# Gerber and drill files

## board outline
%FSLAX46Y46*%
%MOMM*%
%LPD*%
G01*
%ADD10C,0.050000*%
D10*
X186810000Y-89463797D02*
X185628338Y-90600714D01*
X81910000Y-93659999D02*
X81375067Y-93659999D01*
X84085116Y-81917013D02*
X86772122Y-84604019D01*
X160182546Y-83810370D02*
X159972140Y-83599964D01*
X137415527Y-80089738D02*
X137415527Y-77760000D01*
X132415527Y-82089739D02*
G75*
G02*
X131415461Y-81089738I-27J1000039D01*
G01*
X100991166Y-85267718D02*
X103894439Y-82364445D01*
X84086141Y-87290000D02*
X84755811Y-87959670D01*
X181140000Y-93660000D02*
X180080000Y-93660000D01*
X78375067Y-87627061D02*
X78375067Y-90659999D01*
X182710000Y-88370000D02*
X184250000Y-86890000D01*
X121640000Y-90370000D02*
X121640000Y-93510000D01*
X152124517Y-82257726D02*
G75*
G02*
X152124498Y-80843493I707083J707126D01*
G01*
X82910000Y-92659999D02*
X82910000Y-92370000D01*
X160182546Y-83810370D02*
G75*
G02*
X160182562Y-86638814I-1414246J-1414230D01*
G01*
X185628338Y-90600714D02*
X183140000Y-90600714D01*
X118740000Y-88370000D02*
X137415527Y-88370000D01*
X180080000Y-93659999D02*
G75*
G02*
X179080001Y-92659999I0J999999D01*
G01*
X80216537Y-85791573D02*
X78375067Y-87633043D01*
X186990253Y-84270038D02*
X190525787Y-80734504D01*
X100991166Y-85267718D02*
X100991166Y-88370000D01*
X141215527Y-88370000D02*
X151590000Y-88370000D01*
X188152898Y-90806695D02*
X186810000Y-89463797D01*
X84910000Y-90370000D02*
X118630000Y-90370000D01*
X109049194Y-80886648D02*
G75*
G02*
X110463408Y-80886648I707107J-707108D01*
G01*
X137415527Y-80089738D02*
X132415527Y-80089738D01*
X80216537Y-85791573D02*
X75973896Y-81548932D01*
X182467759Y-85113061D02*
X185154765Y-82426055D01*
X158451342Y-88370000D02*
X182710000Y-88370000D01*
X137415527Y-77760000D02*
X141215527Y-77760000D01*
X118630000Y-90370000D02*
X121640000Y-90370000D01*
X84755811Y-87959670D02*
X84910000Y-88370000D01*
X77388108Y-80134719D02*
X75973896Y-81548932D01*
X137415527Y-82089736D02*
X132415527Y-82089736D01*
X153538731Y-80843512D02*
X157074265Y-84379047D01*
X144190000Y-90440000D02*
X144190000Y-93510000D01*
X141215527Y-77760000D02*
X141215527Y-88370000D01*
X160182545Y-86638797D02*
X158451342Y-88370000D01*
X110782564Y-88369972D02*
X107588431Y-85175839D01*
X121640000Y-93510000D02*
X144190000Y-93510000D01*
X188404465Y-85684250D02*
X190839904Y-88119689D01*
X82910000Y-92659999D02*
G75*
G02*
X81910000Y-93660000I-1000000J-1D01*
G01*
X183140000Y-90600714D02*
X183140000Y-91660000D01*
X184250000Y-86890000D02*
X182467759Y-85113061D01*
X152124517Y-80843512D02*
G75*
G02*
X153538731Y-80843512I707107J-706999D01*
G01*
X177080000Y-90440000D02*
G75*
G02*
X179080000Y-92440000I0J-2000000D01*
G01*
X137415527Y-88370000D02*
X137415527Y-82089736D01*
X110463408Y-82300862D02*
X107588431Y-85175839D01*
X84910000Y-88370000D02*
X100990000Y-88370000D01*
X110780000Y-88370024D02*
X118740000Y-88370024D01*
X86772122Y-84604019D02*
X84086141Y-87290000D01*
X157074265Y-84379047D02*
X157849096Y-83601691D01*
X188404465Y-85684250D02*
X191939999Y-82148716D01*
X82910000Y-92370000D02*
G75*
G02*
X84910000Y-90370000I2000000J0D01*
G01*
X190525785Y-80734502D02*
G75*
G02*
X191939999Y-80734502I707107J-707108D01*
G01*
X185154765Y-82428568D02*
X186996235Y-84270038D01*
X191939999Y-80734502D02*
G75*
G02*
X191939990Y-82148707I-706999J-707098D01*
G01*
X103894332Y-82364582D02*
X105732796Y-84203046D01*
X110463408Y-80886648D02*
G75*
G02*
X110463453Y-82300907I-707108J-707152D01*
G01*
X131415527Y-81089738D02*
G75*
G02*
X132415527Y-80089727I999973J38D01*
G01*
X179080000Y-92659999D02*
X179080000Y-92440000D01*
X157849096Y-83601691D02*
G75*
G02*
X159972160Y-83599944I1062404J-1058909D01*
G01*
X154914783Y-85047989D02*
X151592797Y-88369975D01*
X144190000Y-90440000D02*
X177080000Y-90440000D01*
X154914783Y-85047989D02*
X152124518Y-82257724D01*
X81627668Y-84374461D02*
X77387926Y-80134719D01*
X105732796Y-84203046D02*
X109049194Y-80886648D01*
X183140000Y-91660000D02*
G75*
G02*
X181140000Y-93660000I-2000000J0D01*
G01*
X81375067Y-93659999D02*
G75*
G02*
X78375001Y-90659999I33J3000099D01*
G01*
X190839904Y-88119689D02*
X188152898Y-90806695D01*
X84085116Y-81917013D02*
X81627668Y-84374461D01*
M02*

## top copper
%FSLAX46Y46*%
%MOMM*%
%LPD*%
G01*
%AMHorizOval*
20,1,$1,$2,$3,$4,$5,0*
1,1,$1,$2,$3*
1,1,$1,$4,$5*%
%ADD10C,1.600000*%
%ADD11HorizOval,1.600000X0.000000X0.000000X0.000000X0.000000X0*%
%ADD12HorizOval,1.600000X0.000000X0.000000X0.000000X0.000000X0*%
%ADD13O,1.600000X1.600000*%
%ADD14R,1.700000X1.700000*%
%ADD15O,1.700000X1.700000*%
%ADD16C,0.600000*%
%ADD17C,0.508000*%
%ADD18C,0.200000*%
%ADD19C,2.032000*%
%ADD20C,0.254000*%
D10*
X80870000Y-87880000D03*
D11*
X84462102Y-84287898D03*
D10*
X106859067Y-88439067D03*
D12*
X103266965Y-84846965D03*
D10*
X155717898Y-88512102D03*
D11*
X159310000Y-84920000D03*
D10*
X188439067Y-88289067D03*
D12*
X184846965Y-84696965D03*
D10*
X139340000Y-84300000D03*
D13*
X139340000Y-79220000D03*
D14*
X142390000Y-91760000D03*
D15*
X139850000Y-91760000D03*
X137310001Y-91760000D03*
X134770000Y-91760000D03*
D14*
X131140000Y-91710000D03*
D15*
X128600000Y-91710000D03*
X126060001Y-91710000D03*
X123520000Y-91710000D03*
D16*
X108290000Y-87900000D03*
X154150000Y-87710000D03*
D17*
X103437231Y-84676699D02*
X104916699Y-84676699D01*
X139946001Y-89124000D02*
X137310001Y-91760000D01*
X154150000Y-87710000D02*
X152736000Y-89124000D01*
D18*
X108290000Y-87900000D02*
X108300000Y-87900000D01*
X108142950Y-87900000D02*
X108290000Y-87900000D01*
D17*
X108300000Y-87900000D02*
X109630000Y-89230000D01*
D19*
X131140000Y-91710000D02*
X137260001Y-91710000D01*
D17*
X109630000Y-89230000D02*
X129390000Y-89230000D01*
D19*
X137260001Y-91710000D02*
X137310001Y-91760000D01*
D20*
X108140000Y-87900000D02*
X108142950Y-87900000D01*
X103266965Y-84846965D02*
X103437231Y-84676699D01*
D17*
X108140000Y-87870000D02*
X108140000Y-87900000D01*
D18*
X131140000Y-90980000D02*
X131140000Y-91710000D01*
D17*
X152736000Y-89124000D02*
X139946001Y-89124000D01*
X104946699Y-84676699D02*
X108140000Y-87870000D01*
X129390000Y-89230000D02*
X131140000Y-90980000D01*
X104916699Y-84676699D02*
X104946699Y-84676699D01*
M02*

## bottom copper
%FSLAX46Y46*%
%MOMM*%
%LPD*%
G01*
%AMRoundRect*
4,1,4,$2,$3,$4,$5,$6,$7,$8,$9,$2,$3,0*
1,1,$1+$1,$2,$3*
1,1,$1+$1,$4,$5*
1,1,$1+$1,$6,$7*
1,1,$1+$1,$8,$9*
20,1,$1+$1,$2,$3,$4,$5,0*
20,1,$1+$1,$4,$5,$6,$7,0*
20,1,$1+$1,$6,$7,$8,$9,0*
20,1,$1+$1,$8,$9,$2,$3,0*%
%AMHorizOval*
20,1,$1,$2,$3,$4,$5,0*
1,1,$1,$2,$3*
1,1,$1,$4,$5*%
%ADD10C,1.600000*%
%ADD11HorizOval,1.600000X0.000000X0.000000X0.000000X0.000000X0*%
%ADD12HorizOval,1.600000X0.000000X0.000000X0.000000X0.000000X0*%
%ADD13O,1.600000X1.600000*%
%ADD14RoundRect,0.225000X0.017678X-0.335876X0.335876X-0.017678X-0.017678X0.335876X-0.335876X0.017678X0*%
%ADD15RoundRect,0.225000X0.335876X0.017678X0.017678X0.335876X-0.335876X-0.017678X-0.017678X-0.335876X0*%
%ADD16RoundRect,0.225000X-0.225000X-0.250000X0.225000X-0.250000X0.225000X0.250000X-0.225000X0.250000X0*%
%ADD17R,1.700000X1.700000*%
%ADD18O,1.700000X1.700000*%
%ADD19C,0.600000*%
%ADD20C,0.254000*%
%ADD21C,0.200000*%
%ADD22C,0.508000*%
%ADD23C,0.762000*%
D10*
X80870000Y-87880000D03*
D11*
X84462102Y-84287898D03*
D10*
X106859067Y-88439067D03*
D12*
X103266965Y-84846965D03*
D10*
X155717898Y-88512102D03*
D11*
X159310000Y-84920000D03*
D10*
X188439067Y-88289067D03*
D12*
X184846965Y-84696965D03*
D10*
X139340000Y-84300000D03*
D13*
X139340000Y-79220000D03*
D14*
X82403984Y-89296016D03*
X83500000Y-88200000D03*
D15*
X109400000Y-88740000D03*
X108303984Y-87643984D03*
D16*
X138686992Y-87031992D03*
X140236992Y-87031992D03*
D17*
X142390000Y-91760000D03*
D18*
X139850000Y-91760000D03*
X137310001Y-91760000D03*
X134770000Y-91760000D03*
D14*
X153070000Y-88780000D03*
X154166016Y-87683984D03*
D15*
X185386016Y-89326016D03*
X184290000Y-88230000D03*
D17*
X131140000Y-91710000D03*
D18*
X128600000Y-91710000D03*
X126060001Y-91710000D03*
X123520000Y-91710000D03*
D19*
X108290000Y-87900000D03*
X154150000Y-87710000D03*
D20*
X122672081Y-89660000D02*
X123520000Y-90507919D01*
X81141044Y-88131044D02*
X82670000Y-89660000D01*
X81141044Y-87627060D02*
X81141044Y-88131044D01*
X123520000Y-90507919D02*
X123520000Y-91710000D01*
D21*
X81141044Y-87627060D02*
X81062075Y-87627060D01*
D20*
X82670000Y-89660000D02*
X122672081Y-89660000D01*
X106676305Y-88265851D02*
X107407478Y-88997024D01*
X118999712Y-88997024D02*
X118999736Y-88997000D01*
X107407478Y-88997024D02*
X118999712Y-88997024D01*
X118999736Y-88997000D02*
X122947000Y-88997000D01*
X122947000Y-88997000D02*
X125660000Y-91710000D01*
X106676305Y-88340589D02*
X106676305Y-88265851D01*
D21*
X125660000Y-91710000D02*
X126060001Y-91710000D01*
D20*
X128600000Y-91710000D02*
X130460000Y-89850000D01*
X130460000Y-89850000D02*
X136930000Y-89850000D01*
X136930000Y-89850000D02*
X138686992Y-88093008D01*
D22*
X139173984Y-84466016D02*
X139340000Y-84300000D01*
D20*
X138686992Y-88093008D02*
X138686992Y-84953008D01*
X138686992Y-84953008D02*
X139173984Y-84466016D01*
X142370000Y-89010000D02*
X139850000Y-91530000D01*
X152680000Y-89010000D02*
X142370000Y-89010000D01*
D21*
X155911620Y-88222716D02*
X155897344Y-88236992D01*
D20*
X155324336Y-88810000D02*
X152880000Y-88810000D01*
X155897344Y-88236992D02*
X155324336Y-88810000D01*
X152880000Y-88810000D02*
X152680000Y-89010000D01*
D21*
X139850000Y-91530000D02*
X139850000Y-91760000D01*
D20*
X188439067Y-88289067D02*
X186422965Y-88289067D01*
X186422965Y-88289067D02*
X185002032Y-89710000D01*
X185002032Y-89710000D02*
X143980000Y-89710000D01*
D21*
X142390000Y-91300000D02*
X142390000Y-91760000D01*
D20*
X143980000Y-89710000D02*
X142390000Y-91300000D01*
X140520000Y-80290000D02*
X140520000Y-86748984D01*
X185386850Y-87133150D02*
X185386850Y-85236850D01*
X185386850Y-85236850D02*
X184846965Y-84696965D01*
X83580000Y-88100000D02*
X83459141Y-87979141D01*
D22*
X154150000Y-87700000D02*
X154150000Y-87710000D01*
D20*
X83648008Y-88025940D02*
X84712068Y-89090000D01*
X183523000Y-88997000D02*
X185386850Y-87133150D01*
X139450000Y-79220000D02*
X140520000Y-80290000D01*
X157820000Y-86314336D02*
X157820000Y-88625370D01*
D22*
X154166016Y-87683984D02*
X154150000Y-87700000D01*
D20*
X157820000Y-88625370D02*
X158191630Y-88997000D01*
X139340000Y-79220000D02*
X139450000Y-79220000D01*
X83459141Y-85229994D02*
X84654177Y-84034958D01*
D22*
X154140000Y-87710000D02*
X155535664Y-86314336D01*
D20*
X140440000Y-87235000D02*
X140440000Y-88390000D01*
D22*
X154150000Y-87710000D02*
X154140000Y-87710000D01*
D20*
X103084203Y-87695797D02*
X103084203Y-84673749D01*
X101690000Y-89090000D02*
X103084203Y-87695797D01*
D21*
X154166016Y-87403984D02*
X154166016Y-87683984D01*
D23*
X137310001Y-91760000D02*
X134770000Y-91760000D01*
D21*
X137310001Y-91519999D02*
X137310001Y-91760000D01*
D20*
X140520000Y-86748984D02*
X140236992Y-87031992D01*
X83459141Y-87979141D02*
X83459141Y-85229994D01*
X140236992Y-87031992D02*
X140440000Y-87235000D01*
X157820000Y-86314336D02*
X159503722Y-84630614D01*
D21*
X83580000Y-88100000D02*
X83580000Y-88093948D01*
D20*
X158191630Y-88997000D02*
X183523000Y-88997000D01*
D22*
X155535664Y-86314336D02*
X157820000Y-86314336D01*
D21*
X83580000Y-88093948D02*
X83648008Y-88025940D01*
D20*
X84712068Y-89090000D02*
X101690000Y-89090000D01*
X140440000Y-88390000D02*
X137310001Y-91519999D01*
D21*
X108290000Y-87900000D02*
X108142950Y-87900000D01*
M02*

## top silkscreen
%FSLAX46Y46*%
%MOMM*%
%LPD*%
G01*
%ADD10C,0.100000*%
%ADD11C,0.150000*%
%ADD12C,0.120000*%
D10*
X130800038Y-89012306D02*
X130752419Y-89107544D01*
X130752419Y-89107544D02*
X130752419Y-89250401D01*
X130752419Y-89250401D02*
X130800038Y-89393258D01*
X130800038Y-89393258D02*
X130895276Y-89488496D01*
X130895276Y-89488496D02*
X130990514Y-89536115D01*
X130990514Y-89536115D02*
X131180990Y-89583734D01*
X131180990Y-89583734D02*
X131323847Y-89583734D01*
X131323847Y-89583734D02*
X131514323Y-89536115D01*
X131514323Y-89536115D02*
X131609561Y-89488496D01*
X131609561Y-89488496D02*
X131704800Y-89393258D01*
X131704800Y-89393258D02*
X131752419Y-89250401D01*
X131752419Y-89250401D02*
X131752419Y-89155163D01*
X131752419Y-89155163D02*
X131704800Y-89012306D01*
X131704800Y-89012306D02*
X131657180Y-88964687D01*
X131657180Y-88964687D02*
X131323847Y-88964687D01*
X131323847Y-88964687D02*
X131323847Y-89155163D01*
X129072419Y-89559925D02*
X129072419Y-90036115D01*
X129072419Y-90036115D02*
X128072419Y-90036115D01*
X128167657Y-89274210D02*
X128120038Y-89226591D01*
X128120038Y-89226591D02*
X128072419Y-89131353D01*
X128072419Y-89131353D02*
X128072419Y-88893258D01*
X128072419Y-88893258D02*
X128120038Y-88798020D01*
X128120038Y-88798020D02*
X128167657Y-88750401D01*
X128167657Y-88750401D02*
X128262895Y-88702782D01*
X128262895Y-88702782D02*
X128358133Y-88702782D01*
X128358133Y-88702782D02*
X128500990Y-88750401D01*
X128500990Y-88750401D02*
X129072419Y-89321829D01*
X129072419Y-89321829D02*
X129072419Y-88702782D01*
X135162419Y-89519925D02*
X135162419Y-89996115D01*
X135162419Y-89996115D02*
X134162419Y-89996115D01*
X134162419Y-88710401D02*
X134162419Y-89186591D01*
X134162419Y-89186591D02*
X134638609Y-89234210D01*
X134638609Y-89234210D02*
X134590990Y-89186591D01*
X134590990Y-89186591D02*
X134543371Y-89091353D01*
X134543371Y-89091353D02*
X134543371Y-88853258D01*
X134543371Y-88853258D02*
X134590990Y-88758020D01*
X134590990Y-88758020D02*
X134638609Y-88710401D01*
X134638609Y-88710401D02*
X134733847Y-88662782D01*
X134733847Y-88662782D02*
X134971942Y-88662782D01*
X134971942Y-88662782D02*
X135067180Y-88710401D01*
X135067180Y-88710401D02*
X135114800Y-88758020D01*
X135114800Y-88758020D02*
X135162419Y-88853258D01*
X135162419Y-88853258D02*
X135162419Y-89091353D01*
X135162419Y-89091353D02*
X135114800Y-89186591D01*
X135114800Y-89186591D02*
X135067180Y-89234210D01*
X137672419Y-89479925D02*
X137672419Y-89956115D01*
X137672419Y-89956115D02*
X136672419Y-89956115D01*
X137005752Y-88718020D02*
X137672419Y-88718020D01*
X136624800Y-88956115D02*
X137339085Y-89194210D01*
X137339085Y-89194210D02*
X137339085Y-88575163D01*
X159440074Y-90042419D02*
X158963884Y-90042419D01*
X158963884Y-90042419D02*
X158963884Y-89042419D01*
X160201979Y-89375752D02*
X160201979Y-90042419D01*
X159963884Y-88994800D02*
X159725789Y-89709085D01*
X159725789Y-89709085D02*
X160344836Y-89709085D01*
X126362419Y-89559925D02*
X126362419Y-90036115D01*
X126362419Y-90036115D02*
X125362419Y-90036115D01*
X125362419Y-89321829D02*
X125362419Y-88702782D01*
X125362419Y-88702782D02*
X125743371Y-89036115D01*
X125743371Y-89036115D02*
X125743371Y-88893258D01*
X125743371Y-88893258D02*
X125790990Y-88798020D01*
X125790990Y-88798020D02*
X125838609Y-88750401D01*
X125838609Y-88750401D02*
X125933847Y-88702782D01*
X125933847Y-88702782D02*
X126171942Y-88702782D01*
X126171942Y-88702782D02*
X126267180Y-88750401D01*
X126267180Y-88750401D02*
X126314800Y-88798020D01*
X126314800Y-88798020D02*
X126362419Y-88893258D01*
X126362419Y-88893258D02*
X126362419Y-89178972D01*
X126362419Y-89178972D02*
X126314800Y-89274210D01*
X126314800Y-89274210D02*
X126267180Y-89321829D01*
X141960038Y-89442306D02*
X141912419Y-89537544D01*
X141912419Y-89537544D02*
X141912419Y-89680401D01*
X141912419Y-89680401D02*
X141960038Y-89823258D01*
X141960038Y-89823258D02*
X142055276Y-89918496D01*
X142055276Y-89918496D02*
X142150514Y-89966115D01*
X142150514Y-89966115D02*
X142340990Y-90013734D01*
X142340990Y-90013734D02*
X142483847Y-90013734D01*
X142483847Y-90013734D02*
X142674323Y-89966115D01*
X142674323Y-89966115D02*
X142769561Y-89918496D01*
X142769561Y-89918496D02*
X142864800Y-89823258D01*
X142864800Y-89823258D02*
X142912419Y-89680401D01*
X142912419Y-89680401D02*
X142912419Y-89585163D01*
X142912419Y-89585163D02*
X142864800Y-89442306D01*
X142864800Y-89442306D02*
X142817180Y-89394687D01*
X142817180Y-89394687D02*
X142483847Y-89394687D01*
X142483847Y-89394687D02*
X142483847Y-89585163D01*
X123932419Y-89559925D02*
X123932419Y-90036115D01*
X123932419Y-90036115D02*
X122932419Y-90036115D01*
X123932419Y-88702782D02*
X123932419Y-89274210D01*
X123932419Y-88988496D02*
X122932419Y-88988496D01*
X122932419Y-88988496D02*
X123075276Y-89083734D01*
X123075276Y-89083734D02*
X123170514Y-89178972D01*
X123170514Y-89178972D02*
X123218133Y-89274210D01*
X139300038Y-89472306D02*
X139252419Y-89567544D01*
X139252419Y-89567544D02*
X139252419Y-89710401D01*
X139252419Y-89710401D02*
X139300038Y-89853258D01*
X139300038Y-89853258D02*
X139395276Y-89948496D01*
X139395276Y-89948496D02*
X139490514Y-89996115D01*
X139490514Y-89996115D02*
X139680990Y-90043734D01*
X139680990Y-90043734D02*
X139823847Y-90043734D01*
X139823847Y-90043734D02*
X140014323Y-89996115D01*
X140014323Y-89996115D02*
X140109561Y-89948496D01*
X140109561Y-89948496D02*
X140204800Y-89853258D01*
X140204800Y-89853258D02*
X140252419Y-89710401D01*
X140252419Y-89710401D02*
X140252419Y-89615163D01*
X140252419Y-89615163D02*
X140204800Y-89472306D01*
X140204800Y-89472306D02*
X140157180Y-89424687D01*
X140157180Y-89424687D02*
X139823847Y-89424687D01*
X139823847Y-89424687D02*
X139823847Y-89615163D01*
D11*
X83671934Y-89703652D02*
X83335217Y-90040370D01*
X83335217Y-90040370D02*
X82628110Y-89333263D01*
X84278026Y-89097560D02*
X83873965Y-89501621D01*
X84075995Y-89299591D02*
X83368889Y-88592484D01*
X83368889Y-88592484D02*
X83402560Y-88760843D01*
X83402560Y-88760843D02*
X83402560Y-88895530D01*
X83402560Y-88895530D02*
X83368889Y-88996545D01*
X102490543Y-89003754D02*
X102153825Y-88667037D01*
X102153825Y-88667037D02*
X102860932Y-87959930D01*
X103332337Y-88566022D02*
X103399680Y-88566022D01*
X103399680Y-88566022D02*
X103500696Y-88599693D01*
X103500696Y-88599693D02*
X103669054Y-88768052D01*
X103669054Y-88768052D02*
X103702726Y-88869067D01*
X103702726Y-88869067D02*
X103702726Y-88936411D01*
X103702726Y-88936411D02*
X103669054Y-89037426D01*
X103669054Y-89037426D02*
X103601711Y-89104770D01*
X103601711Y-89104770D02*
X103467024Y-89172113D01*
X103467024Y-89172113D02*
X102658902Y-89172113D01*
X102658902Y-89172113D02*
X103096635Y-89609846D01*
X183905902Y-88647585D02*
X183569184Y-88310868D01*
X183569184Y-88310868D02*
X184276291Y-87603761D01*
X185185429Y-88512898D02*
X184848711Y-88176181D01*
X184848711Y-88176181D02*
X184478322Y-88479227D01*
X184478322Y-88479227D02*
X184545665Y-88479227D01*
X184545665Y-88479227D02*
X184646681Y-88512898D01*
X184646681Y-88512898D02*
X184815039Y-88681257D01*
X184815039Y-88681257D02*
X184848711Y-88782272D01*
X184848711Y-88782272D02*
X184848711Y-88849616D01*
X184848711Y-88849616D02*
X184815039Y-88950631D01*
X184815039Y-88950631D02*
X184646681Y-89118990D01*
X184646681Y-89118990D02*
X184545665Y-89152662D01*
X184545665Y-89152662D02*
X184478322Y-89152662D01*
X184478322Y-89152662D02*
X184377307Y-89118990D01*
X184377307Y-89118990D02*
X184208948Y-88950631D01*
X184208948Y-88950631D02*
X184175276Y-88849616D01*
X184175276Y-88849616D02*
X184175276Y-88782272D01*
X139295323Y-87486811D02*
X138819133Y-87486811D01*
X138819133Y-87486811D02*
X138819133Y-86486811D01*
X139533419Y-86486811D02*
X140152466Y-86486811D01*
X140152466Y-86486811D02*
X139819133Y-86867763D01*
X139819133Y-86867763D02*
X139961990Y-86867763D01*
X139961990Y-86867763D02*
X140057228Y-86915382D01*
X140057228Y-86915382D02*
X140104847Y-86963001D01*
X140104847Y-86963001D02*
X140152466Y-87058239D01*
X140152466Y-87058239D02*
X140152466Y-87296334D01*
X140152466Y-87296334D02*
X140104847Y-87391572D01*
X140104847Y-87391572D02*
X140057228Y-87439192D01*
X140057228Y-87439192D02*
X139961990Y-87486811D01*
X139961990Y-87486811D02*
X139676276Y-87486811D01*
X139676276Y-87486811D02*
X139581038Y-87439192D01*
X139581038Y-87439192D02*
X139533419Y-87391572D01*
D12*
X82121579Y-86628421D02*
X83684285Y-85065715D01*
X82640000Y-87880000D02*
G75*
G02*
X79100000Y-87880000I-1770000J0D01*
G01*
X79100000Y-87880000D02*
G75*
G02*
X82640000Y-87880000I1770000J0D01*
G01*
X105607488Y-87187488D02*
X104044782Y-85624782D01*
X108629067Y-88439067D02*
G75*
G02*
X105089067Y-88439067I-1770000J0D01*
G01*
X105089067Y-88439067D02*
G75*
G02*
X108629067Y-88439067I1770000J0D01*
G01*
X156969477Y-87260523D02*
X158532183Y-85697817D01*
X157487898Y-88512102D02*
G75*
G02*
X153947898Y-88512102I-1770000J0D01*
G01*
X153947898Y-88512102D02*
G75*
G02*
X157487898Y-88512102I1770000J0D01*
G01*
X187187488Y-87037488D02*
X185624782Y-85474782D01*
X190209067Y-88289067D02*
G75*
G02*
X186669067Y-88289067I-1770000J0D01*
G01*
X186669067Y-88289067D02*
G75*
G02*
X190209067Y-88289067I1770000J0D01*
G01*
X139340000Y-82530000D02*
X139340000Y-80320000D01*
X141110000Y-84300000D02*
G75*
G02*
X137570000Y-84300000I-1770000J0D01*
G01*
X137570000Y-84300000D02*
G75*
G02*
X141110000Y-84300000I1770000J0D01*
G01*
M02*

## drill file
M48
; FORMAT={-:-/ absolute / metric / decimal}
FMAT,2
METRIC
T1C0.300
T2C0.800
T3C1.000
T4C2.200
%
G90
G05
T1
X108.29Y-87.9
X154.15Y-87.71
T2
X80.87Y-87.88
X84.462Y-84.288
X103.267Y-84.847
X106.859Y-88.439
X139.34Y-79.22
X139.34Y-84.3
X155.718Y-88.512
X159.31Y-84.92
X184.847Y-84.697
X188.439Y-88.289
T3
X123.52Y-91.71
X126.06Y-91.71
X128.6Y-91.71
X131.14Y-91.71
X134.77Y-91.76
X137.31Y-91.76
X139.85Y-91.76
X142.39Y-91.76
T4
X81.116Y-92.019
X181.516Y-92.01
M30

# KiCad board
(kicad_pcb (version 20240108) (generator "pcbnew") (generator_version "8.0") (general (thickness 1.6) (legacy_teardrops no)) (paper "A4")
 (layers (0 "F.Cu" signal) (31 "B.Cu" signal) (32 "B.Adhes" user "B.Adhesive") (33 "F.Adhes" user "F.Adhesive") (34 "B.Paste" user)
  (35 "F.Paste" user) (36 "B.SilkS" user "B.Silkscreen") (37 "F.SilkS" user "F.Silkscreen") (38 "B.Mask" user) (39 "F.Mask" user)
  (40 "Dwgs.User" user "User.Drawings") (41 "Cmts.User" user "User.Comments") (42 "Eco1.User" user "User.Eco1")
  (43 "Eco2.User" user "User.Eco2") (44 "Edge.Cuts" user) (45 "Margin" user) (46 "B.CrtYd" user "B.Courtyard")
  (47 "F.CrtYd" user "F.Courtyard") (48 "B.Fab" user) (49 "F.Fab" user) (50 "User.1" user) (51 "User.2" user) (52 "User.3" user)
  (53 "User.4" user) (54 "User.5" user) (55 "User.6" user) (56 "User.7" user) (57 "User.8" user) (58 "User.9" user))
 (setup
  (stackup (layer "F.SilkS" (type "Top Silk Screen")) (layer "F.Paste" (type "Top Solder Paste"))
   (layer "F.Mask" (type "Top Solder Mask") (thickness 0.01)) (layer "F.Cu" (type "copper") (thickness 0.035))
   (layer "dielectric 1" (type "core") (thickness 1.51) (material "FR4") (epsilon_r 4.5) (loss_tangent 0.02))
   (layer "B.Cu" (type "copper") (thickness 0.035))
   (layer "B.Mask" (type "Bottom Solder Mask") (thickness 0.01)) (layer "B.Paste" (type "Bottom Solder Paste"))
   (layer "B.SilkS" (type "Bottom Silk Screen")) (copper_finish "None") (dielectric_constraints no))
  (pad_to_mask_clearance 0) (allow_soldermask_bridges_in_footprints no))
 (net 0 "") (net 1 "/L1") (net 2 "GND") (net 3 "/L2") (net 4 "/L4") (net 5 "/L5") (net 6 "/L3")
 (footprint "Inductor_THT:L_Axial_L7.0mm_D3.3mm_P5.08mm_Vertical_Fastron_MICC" (layer "F.Cu") (at 80.87 87.88 45)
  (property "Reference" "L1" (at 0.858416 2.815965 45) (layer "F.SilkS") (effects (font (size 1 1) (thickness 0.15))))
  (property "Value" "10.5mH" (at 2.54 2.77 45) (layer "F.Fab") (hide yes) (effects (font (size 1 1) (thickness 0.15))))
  (fp_line (start 1.77 0) (end 3.98 0) (stroke (width 0.12) (type solid)) (layer "F.SilkS"))
  (fp_circle (center 0 0) (end 1.77 0) (stroke (width 0.12) (type solid)) (fill none) (layer "F.SilkS"))
  (pad "1" thru_hole circle (at 0 0 45) (size 1.6 1.6) (drill 0.8) (layers "*.Cu" "*.Mask") (remove_unused_layers no) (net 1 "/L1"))
  (pad "2" thru_hole oval (at 5.079999 0 45) (size 1.6 1.6) (drill 0.8) (layers "*.Cu" "*.Mask") (remove_unused_layers no) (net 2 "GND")))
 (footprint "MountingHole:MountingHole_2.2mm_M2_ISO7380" (layer "F.Cu") (at 81.115528 92.019237)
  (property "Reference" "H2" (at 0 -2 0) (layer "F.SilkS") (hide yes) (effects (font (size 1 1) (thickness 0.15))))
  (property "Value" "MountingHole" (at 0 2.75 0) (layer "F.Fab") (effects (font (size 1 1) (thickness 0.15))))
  (pad "" np_thru_hole circle (at 0 0) (size 2.2 2.2) (drill 2.2) (layers "*.Cu" "*.Mask")))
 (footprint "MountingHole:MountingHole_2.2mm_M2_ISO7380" (layer "F.Cu") (at 181.515528 92.01)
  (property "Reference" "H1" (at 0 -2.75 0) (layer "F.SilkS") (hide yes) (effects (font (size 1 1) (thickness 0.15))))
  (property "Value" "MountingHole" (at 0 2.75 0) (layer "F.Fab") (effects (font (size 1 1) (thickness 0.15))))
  (pad "" np_thru_hole circle (at 0 0) (size 2.2 2.2) (drill 2.2) (layers "*.Cu" "*.Mask")))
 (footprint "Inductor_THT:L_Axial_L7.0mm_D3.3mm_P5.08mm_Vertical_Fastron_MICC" (layer "F.Cu") (at 106.859067 88.439067 135)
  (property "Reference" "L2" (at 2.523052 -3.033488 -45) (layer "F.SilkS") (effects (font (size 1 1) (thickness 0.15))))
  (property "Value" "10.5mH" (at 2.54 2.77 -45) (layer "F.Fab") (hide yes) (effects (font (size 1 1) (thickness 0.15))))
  (fp_line (start 1.77 0) (end 3.98 0) (stroke (width 0.12) (type solid)) (layer "F.SilkS"))
  (fp_circle (center 0 0) (end 1.77 0) (stroke (width 0.12) (type solid)) (fill none) (layer "F.SilkS"))
  (pad "1" thru_hole circle (at 0 0 135) (size 1.6 1.6) (drill 0.8) (layers "*.Cu" "*.Mask") (remove_unused_layers no) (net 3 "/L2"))
  (pad "2" thru_hole oval (at 5.079999 0 135) (size 1.6 1.6) (drill 0.8) (layers "*.Cu" "*.Mask") (remove_unused_layers no) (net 2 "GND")))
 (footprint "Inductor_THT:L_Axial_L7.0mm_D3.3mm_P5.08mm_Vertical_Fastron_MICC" (layer "F.Cu") (at 155.717898 88.512102 45)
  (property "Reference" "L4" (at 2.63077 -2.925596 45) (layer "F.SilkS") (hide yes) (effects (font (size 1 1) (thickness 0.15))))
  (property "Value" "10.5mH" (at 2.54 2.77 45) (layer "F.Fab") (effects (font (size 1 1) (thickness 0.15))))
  (fp_line (start 1.77 0) (end 3.98 0) (stroke (width 0.12) (type solid)) (layer "F.SilkS"))
  (fp_circle (center 0 0) (end 1.77 0) (stroke (width 0.12) (type solid)) (fill none) (layer "F.SilkS"))
  (pad "1" thru_hole circle (at 0 0 45) (size 1.6 1.6) (drill 0.8) (layers "*.Cu" "*.Mask") (remove_unused_layers no) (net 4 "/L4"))
  (pad "2" thru_hole oval (at 5.079999 0 45) (size 1.6 1.6) (drill 0.8) (layers "*.Cu" "*.Mask") (remove_unused_layers no) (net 2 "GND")))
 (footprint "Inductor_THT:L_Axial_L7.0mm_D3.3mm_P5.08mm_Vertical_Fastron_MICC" (layer "F.Cu") (at 188.439067 88.289067 135)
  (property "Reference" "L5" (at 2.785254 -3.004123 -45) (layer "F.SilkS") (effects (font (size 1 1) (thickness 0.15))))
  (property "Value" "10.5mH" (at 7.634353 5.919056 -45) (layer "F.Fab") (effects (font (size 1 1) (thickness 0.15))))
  (fp_line (start 1.77 0) (end 3.98 0) (stroke (width 0.12) (type solid)) (layer "F.SilkS"))
  (fp_circle (center 0 0) (end 1.77 0) (stroke (width 0.12) (type solid)) (fill none) (layer "F.SilkS"))
  (pad "1" thru_hole circle (at 0 0 135) (size 1.6 1.6) (drill 0.8) (layers "*.Cu" "*.Mask") (remove_unused_layers no) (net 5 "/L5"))
  (pad "2" thru_hole oval (at 5.079999 0 135) (size 1.6 1.6) (drill 0.8) (layers "*.Cu" "*.Mask") (remove_unused_layers no) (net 2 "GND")))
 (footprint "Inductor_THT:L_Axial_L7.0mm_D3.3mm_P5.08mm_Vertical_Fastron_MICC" (layer "F.Cu") (at 139.34 84.3 90)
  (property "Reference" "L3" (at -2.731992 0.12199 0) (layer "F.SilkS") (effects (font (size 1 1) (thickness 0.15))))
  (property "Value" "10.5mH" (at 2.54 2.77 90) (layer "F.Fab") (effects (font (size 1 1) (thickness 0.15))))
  (fp_line (start 1.77 0) (end 3.98 0) (stroke (width 0.12) (type solid)) (layer "F.SilkS"))
  (fp_circle (center 0 0) (end 1.77 0) (stroke (width 0.12) (type solid)) (fill none) (layer "F.SilkS"))
  (pad "1" thru_hole circle (at 0 0 90) (size 1.6 1.6) (drill 0.8) (layers "*.Cu" "*.Mask") (remove_unused_layers no) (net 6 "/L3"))
  (pad "2" thru_hole oval (at 5.08 0 90) (size 1.6 1.6) (drill 0.8) (layers "*.Cu" "*.Mask") (remove_unused_layers no) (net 2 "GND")))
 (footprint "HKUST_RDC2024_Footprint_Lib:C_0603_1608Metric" (layer "B.Cu") (at 82.951992 88.748008 45)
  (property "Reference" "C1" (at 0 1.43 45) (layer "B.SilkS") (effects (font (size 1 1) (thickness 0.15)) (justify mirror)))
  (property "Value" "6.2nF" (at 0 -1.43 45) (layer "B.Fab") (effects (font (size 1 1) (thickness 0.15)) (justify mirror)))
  (pad "1" smd roundrect (at -0.775 0 45) (size 0.9 0.95) (layers "B.Cu" "B.Paste" "B.Mask") (roundrect_rratio 0.25) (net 1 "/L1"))
  (pad "2" smd roundrect (at 0.775 0 45) (size 0.9 0.95) (layers "B.Cu" "B.Paste" "B.Mask") (roundrect_rratio 0.25) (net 2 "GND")))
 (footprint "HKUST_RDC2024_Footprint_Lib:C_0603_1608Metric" (layer "B.Cu") (at 108.851992 88.191992 135)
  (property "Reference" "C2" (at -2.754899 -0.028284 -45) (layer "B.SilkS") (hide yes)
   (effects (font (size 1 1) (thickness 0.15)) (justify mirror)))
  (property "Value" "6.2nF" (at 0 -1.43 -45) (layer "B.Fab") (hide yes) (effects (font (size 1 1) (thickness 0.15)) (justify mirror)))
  (pad "1" smd roundrect (at -0.775 0 135) (size 0.9 0.95) (layers "B.Cu" "B.Paste" "B.Mask") (roundrect_rratio 0.25) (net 3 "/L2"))
  (pad "2" smd roundrect (at 0.775 0 135) (size 0.9 0.95) (layers "B.Cu" "B.Paste" "B.Mask") (roundrect_rratio 0.25) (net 2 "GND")))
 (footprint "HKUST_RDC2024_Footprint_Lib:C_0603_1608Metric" (layer "B.Cu") (at 139.461992 87.031992)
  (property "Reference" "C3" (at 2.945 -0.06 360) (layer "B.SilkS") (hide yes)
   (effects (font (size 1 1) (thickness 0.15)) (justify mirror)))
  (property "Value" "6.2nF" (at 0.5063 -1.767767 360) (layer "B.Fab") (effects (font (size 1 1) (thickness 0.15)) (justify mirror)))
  (pad "1" smd roundrect (at -0.775 0) (size 0.9 0.95) (layers "B.Cu" "B.Paste" "B.Mask") (roundrect_rratio 0.25) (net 6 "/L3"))
  (pad "2" smd roundrect (at 0.775 0) (size 0.9 0.95) (layers "B.Cu" "B.Paste" "B.Mask") (roundrect_rratio 0.25) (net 2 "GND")))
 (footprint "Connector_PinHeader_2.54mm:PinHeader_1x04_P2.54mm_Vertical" (layer "B.Cu") (at 142.39 91.76 90)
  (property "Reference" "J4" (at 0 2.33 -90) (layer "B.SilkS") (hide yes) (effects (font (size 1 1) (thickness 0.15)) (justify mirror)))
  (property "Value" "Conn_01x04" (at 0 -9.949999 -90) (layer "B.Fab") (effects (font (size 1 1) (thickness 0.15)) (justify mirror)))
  (pad "1" thru_hole rect (at 0 0 90) (size 1.7 1.7) (drill 1) (layers "*.Cu" "*.Mask") (remove_unused_layers no) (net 5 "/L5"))
  (pad "2" thru_hole oval (at 0 -2.54 90) (size 1.7 1.7) (drill 1) (layers "*.Cu" "*.Mask") (remove_unused_layers no) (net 4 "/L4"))
  (pad "3" thru_hole oval (at 0 -5.079999 90) (size 1.7 1.7) (drill 1) (layers "*.Cu" "*.Mask") (remove_unused_layers no) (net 2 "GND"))
  (pad "4" thru_hole oval (at 0 -7.62 90) (size 1.7 1.7) (drill 1) (layers "*.Cu" "*.Mask") (remove_unused_layers no) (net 2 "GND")))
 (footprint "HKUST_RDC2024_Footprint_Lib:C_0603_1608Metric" (layer "B.Cu") (at 153.618008 88.231992 45)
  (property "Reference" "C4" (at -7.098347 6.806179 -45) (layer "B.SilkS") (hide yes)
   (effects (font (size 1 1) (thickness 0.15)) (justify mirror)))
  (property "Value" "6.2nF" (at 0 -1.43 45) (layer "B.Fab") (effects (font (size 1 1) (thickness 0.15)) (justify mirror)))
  (pad "1" smd roundrect (at -0.775 0 45) (size 0.9 0.95) (layers "B.Cu" "B.Paste" "B.Mask") (roundrect_rratio 0.25) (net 4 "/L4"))
  (pad "2" smd roundrect (at 0.775 0 45) (size 0.9 0.95) (layers "B.Cu" "B.Paste" "B.Mask") (roundrect_rratio 0.25) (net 2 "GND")))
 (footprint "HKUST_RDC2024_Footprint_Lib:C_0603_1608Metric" (layer "B.Cu") (at 184.838008 88.778008 135)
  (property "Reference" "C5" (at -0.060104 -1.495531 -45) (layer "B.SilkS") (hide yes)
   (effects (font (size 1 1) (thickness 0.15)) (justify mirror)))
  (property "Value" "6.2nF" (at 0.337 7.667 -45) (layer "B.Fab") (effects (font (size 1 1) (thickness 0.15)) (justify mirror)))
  (pad "1" smd roundrect (at -0.775 0 135) (size 0.9 0.95) (layers "B.Cu" "B.Paste" "B.Mask") (roundrect_rratio 0.25) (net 5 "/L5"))
  (pad "2" smd roundrect (at 0.775 0 135) (size 0.9 0.95) (layers "B.Cu" "B.Paste" "B.Mask") (roundrect_rratio 0.25) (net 2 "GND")))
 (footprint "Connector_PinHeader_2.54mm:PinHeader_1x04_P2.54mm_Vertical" (layer "B.Cu") (at 131.14 91.71 90)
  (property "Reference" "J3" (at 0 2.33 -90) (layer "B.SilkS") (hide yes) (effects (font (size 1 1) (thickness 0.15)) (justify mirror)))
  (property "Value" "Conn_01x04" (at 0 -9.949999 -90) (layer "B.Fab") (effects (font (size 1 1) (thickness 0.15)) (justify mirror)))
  (pad "1" thru_hole rect (at 0 0 90) (size 1.7 1.7) (drill 1) (layers "*.Cu" "*.Mask") (remove_unused_layers no) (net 2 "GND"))
  (pad "2" thru_hole oval (at 0 -2.54 90) (size 1.7 1.7) (drill 1) (layers "*.Cu" "*.Mask") (remove_unused_layers no) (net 6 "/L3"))
  (pad "3" thru_hole oval (at 0 -5.079999 90) (size 1.7 1.7) (drill 1) (layers "*.Cu" "*.Mask") (remove_unused_layers no) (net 3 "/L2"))
  (pad "4" thru_hole oval (at 0 -7.62 90) (size 1.7 1.7) (drill 1) (layers "*.Cu" "*.Mask") (remove_unused_layers no) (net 1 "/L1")))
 (gr_line (start 186.81 89.463797) (end 185.628338 90.600714) (stroke (width 0.05) (type default)) (layer "Edge.Cuts"))
 (gr_line (start 81.91 93.659999) (end 81.375067 93.659999) (stroke (width 0.05) (type default)) (layer "Edge.Cuts"))
 (gr_line (start 84.085116 81.917013) (end 86.772122 84.604019) (stroke (width 0.05) (type default)) (layer "Edge.Cuts"))
 (gr_line (start 160.182546 83.81037) (end 159.97214 83.599964) (stroke (width 0.05) (type default)) (layer "Edge.Cuts"))
 (gr_line (start 137.415527 80.089738) (end 137.415527 77.76) (stroke (width 0.05) (type default)) (layer "Edge.Cuts"))
 (gr_arc (start 132.415527 82.089739) (mid 131.70842 81.796845) (end 131.415527 81.089738) (stroke (width 0.05) (type default))
  (layer "Edge.Cuts"))
 (gr_line (start 100.991166 85.267718) (end 103.894439 82.364445) (stroke (width 0.05) (type default)) (layer "Edge.Cuts"))
 (gr_line (start 84.086141 87.29) (end 84.755811 87.95967) (stroke (width 0.05) (type default)) (layer "Edge.Cuts"))
 (gr_line (start 181.14 93.66) (end 180.08 93.66) (stroke (width 0.05) (type default)) (layer "Edge.Cuts"))
 (gr_line (start 78.375067 87.627061) (end 78.375067 90.659999) (stroke (width 0.05) (type default)) (layer "Edge.Cuts"))
 (gr_line (start 182.71 88.37) (end 184.25 86.89) (stroke (width 0.05) (type default)) (layer "Edge.Cuts"))
 (gr_line (start 121.64 90.37) (end 121.64 93.51) (stroke (width 0.05) (type default)) (layer "Edge.Cuts"))
 (gr_arc (start 152.124517 82.257726) (mid 151.831624 81.550619) (end 152.124517 80.843512) (stroke (width 0.05) (type default))
  (layer "Edge.Cuts"))
 (gr_line (start 82.91 92.659999) (end 82.91 92.37) (stroke (width 0.05) (type default)) (layer "Edge.Cuts"))
 (gr_arc (start 160.182546 83.81037) (mid 160.768332 85.224584) (end 160.182545 86.638797) (stroke (width 0.05) (type default))
  (layer "Edge.Cuts"))
 (gr_line (start 185.628338 90.600714) (end 183.14 90.600714) (stroke (width 0.05) (type default)) (layer "Edge.Cuts"))
 (gr_line (start 118.74 88.37) (end 137.415527 88.37) (stroke (width 0.05) (type default)) (layer "Edge.Cuts"))
 (gr_arc (start 180.08 93.659999) (mid 179.372893 93.367106) (end 179.08 92.659999) (stroke (width 0.05) (type default)) (layer "Edge.Cuts"))
 (gr_line (start 80.216537 85.791573) (end 78.375067 87.633043) (stroke (width 0.05) (type default)) (layer "Edge.Cuts"))
 (gr_line (start 186.990253 84.270038) (end 190.525787 80.734504) (stroke (width 0.05) (type default)) (layer "Edge.Cuts"))
 (gr_line (start 100.991166 85.267718) (end 100.991166 88.37) (stroke (width 0.05) (type default)) (layer "Edge.Cuts"))
 (gr_line (start 141.215527 88.37) (end 151.59 88.37) (stroke (width 0.05) (type default)) (layer "Edge.Cuts"))
 (gr_line (start 188.152898 90.806695) (end 186.81 89.463797) (stroke (width 0.05) (type default)) (layer "Edge.Cuts"))
 (gr_line (start 84.91 90.37) (end 118.63 90.37) (stroke (width 0.05) (type default)) (layer "Edge.Cuts"))
 (gr_arc (start 109.049194 80.886648) (mid 109.756301 80.593755) (end 110.463408 80.886648) (stroke (width 0.05) (type default))
  (layer "Edge.Cuts"))
 (gr_line (start 137.415527 80.089738) (end 132.415527 80.089738) (stroke (width 0.05) (type default)) (layer "Edge.Cuts"))
 (gr_line (start 80.216537 85.791573) (end 75.973896 81.548932) (stroke (width 0.05) (type default)) (layer "Edge.Cuts"))
 (gr_line (start 182.467759 85.113061) (end 185.154765 82.426055) (stroke (width 0.05) (type default)) (layer "Edge.Cuts"))
 (gr_line (start 158.451342 88.37) (end 182.71 88.37) (stroke (width 0.05) (type default)) (layer "Edge.Cuts"))
 (gr_line (start 137.415527 77.76) (end 141.215527 77.76) (stroke (width 0.05) (type default)) (layer "Edge.Cuts"))
 (gr_line (start 118.63 90.37) (end 121.64 90.37) (stroke (width 0.05) (type default)) (layer "Edge.Cuts"))
 (gr_line (start 84.755811 87.95967) (end 84.91 88.37) (stroke (width 0.05) (type default)) (layer "Edge.Cuts"))
 (gr_line (start 77.388108 80.134719) (end 75.973896 81.548932) (stroke (width 0.05) (type default)) (layer "Edge.Cuts"))
 (gr_line (start 137.415527 82.089736) (end 132.415527 82.089736) (stroke (width 0.05) (type default)) (layer "Edge.Cuts"))
 (gr_line (start 153.538731 80.843512) (end 157.074265 84.379047) (stroke (width 0.05) (type default)) (layer "Edge.Cuts"))
 (gr_line (start 144.19 90.44) (end 144.19 93.51) (stroke (width 0.05) (type default)) (layer "Edge.Cuts"))
 (gr_line (start 141.215527 77.76) (end 141.215527 88.37) (stroke (width 0.05) (type default)) (layer "Edge.Cuts"))
 (gr_line (start 160.182545 86.638797) (end 158.451342 88.37) (stroke (width 0.05) (type default)) (layer "Edge.Cuts"))
 (gr_line (start 110.782564 88.369972) (end 107.588431 85.175839) (stroke (width 0.05) (type default)) (layer "Edge.Cuts"))
 (gr_line (start 121.64 93.51) (end 144.19 93.51) (stroke (width 0.05) (type default)) (layer "Edge.Cuts"))
 (gr_line (start 188.404465 85.68425) (end 190.839904 88.119689) (stroke (width 0.05) (type default)) (layer "Edge.Cuts"))
 (gr_arc (start 82.91 92.659999) (mid 82.617107 93.367106) (end 81.91 93.659999) (stroke (width 0.05) (type default)) (layer "Edge.Cuts"))
 (gr_line (start 183.14 90.600714) (end 183.14 91.66) (stroke (width 0.05) (type default)) (layer "Edge.Cuts"))
 (gr_line (start 184.25 86.89) (end 182.467759 85.113061) (stroke (width 0.05) (type default)) (layer "Edge.Cuts"))
 (gr_arc (start 152.124517 80.843512) (mid 152.831637 80.550587) (end 153.538731 80.843512) (stroke (width 0.05) (type default))
  (layer "Edge.Cuts"))
 (gr_arc (start 177.08 90.44) (mid 178.494214 91.025786) (end 179.08 92.44) (stroke (width 0.05) (type default)) (layer "Edge.Cuts"))
 (gr_line (start 137.415527 88.37) (end 137.415527 82.089736) (stroke (width 0.05) (type default)) (layer "Edge.Cuts"))
 (gr_line (start 110.463408 82.300862) (end 107.588431 85.175839) (stroke (width 0.05) (type default)) (layer "Edge.Cuts"))
 (gr_line (start 84.91 88.37) (end 100.99 88.37) (stroke (width 0.05) (type default)) (layer "Edge.Cuts"))
 (gr_line (start 110.78 88.370024) (end 118.74 88.370024) (stroke (width 0.05) (type default)) (layer "Edge.Cuts"))
 (gr_line (start 86.772122 84.604019) (end 84.086141 87.29) (stroke (width 0.05) (type default)) (layer "Edge.Cuts"))
 (gr_line (start 157.074265 84.379047) (end 157.849096 83.601691) (stroke (width 0.05) (type default)) (layer "Edge.Cuts"))
 (gr_line (start 188.404465 85.68425) (end 191.939999 82.148716) (stroke (width 0.05) (type default)) (layer "Edge.Cuts"))
 (gr_arc (start 82.91 92.37) (mid 83.495786 90.955786) (end 84.91 90.37) (stroke (width 0.05) (type default)) (layer "Edge.Cuts"))
 (gr_arc (start 190.525785 80.734502) (mid 191.232892 80.441609) (end 191.939999 80.734502) (stroke (width 0.05) (type default))
  (layer "Edge.Cuts"))
 (gr_line (start 185.154765 82.428568) (end 186.996235 84.270038) (stroke (width 0.05) (type default)) (layer "Edge.Cuts"))
 (gr_arc (start 191.939999 80.734502) (mid 192.232924 81.441622) (end 191.939999 82.148716) (stroke (width 0.05) (type default))
  (layer "Edge.Cuts"))
 (gr_line (start 103.894332 82.364582) (end 105.732796 84.203046) (stroke (width 0.05) (type default)) (layer "Edge.Cuts"))
 (gr_arc (start 110.463408 80.886648) (mid 110.756301 81.593755) (end 110.463408 82.300862) (stroke (width 0.05) (type default))
  (layer "Edge.Cuts"))
 (gr_arc (start 131.415527 81.089738) (mid 131.708407 80.3826) (end 132.415527 80.089738) (stroke (width 0.05) (type default))
  (layer "Edge.Cuts"))
 (gr_line (start 179.08 92.659999) (end 179.08 92.44) (stroke (width 0.05) (type default)) (layer "Edge.Cuts"))
 (gr_arc (start 157.849096 83.601691) (mid 158.91026 83.160625) (end 159.97214 83.599964) (stroke (width 0.05) (type default))
  (layer "Edge.Cuts"))
 (gr_line (start 154.914783 85.047989) (end 151.592797 88.369975) (stroke (width 0.05) (type default)) (layer "Edge.Cuts"))
 (gr_line (start 144.19 90.44) (end 177.08 90.44) (stroke (width 0.05) (type default)) (layer "Edge.Cuts"))
 (gr_line (start 154.914783 85.047989) (end 152.124518 82.257724) (stroke (width 0.05) (type default)) (layer "Edge.Cuts"))
 (gr_line (start 81.627668 84.374461) (end 77.387926 80.134719) (stroke (width 0.05) (type default)) (layer "Edge.Cuts"))
 (gr_line (start 105.732796 84.203046) (end 109.049194 80.886648) (stroke (width 0.05) (type default)) (layer "Edge.Cuts"))
 (gr_arc (start 183.14 91.66) (mid 182.554214 93.074214) (end 181.14 93.66) (stroke (width 0.05) (type default)) (layer "Edge.Cuts"))
 (gr_arc (start 81.375067 93.659999) (mid 79.253768 92.781308) (end 78.375067 90.659999) (stroke (width 0.05) (type default))
  (layer "Edge.Cuts"))
 (gr_line (start 190.839904 88.119689) (end 188.152898 90.806695) (stroke (width 0.05) (type default)) (layer "Edge.Cuts"))
 (gr_line (start 84.085116 81.917013) (end 81.627668 84.374461) (stroke (width 0.05) (type default)) (layer "Edge.Cuts"))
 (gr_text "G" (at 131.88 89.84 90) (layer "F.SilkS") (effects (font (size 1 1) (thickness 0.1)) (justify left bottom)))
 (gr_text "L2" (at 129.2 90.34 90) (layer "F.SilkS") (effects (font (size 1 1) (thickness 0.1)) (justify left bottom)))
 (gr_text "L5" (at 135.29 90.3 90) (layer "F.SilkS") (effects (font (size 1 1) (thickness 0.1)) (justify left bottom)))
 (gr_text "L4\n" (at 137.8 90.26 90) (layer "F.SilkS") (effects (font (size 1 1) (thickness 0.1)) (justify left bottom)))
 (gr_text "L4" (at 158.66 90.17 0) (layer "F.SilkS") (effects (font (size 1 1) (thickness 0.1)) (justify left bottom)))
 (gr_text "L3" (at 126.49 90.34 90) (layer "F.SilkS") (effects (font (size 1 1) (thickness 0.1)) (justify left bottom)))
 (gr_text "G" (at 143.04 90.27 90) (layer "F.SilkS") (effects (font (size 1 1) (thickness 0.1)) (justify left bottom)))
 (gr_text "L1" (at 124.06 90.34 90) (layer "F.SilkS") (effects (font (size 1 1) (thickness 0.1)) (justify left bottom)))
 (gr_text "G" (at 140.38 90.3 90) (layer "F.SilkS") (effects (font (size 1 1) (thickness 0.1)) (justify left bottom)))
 (segment (start 122.672081 89.66) (end 123.52 90.507919) (width 0.254) (layer "B.Cu") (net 1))
 (segment (start 81.141044 88.131044) (end 82.67 89.66) (width 0.254) (layer "B.Cu") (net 1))
 (segment (start 81.141044 87.62706) (end 81.141044 88.131044) (width 0.254) (layer "B.Cu") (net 1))
 (segment (start 123.52 90.507919) (end 123.52 91.71) (width 0.254) (layer "B.Cu") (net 1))
 (segment (start 81.141044 87.62706) (end 81.062075 87.62706) (width 0.2) (layer "B.Cu") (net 1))
 (segment (start 82.67 89.66) (end 122.672081 89.66) (width 0.254) (layer "B.Cu") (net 1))
 (segment (start 106.676305 88.265851) (end 107.407478 88.997024) (width 0.254) (layer "B.Cu") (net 3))
 (segment (start 118.999712 88.997024) (end 118.999736 88.997) (width 0.254) (layer "B.Cu") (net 3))
 (segment (start 107.407478 88.997024) (end 118.999712 88.997024) (width 0.254) (layer "B.Cu") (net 3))
 (segment (start 118.999736 88.997) (end 122.947 88.997) (width 0.254) (layer "B.Cu") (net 3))
 (segment (start 122.947 88.997) (end 125.66 91.71) (width 0.254) (layer "B.Cu") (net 3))
 (segment (start 106.676305 88.340589) (end 106.676305 88.265851) (width 0.254) (layer "B.Cu") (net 3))
 (segment (start 125.66 91.71) (end 126.060001 91.71) (width 0.2) (layer "B.Cu") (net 3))
 (segment (start 128.6 91.71) (end 130.46 89.85) (width 0.254) (layer "B.Cu") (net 6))
 (segment (start 130.46 89.85) (end 136.93 89.85) (width 0.254) (layer "B.Cu") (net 6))
 (segment (start 136.93 89.85) (end 138.686992 88.093008) (width 0.254) (layer "B.Cu") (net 6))
 (segment (start 139.173984 84.466016) (end 139.34 84.3) (width 0.508) (layer "B.Cu") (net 6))
 (segment (start 138.686992 88.093008) (end 138.686992 84.953008) (width 0.254) (layer "B.Cu") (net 6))
 (segment (start 138.686992 84.953008) (end 139.173984 84.466016) (width 0.254) (layer "B.Cu") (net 6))
 (segment (start 142.37 89.01) (end 139.85 91.53) (width 0.254) (layer "B.Cu") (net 4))
 (segment (start 152.68 89.01) (end 142.37 89.01) (width 0.254) (layer "B.Cu") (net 4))
 (segment (start 155.91162 88.222716) (end 155.897344 88.236992) (width 0.2) (layer "B.Cu") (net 4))
 (segment (start 155.324336 88.81) (end 152.88 88.81) (width 0.254) (layer "B.Cu") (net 4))
 (segment (start 155.897344 88.236992) (end 155.324336 88.81) (width 0.254) (layer "B.Cu") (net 4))
 (segment (start 152.88 88.81) (end 152.68 89.01) (width 0.254) (layer "B.Cu") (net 4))
 (segment (start 139.85 91.53) (end 139.85 91.76) (width 0.2) (layer "B.Cu") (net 4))
 (segment (start 188.439067 88.289067) (end 186.422965 88.289067) (width 0.254) (layer "B.Cu") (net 5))
 (segment (start 186.422965 88.289067) (end 185.002032 89.71) (width 0.254) (layer "B.Cu") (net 5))
 (segment (start 185.002032 89.71) (end 143.98 89.71) (width 0.254) (layer "B.Cu") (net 5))
 (segment (start 142.39 91.3) (end 142.39 91.76) (width 0.2) (layer "B.Cu") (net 5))
 (segment (start 143.98 89.71) (end 142.39 91.3) (width 0.254) (layer "B.Cu") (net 5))
 (segment (start 103.437231 84.676699) (end 104.916699 84.676699) (width 0.508) (layer "F.Cu") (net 2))
 (segment (start 139.946001 89.124) (end 137.310001 91.76) (width 0.508) (layer "F.Cu") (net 2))
 (segment (start 154.15 87.71) (end 152.736 89.124) (width 0.508) (layer "F.Cu") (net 2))
 (segment (start 108.29 87.9) (end 108.3 87.9) (width 0.2) (layer "F.Cu") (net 2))
 (segment (start 108.14295 87.9) (end 108.29 87.9) (width 0.2) (layer "F.Cu") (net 2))
 (segment (start 108.3 87.9) (end 109.63 89.23) (width 0.508) (layer "F.Cu") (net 2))
 (segment (start 131.14 91.71) (end 137.260001 91.71) (width 2.032) (layer "F.Cu") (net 2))
 (segment (start 109.63 89.23) (end 129.39 89.23) (width 0.508) (layer "F.Cu") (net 2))
 (segment (start 137.260001 91.71) (end 137.310001 91.76) (width 2.032) (layer "F.Cu") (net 2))
 (segment (start 108.14 87.9) (end 108.14295 87.9) (width 0.254) (layer "F.Cu") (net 2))
 (segment (start 103.266965 84.846965) (end 103.437231 84.676699) (width 0.254) (layer "F.Cu") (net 2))
 (segment (start 108.14 87.87) (end 108.14 87.9) (width 0.508) (layer "F.Cu") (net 2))
 (segment (start 131.14 90.98) (end 131.14 91.71) (width 0.2) (layer "F.Cu") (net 2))
 (segment (start 152.736 89.124) (end 139.946001 89.124) (width 0.508) (layer "F.Cu") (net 2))
 (segment (start 104.946699 84.676699) (end 108.14 87.87) (width 0.508) (layer "F.Cu") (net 2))
 (segment (start 129.39 89.23) (end 131.14 90.98) (width 0.508) (layer "F.Cu") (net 2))
 (segment (start 104.916699 84.676699) (end 104.946699 84.676699) (width 0.508) (layer "F.Cu") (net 2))
 (via (at 108.29 87.9) (size 0.6) (drill 0.3) (layers "F.Cu" "B.Cu") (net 2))
 (via (at 154.15 87.71) (size 0.6) (drill 0.3) (layers "F.Cu" "B.Cu") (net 2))
 (segment (start 140.52 80.29) (end 140.52 86.748984) (width 0.254) (layer "B.Cu") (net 2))
 (segment (start 185.38685 87.13315) (end 185.38685 85.23685) (width 0.254) (layer "B.Cu") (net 2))
 (segment (start 185.38685 85.23685) (end 184.846965 84.696965) (width 0.254) (layer "B.Cu") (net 2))
 (segment (start 83.58 88.1) (end 83.459141 87.979141) (width 0.254) (layer "B.Cu") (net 2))
 (segment (start 154.15 87.7) (end 154.15 87.71) (width 0.508) (layer "B.Cu") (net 2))
 (segment (start 83.648008 88.02594) (end 84.712068 89.09) (width 0.254) (layer "B.Cu") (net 2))
 (segment (start 183.523 88.997) (end 185.38685 87.13315) (width 0.254) (layer "B.Cu") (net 2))
 (segment (start 139.45 79.22) (end 140.52 80.29) (width 0.254) (layer "B.Cu") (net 2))
 (segment (start 157.82 86.314336) (end 157.82 88.62537) (width 0.254) (layer "B.Cu") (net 2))
 (segment (start 154.166016 87.683984) (end 154.15 87.7) (width 0.508) (layer "B.Cu") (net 2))
 (segment (start 157.82 88.62537) (end 158.19163 88.997) (width 0.254) (layer "B.Cu") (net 2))
 (segment (start 139.34 79.22) (end 139.45 79.22) (width 0.254) (layer "B.Cu") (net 2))
 (segment (start 83.459141 85.229994) (end 84.654177 84.034958) (width 0.254) (layer "B.Cu") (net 2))
 (segment (start 154.14 87.71) (end 155.535664 86.314336) (width 0.508) (layer "B.Cu") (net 2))
 (segment (start 140.44 87.235) (end 140.44 88.39) (width 0.254) (layer "B.Cu") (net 2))
 (segment (start 154.15 87.71) (end 154.14 87.71) (width 0.508) (layer "B.Cu") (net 2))
 (segment (start 103.084203 87.695797) (end 103.084203 84.673749) (width 0.254) (layer "B.Cu") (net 2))
 (segment (start 101.69 89.09) (end 103.084203 87.695797) (width 0.254) (layer "B.Cu") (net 2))
 (segment (start 154.166016 87.403984) (end 154.166016 87.683984) (width 0.2) (layer "B.Cu") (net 2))
 (segment (start 137.310001 91.76) (end 134.77 91.76) (width 0.762) (layer "B.Cu") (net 2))
 (segment (start 137.310001 91.519999) (end 137.310001 91.76) (width 0.2) (layer "B.Cu") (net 2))
 (segment (start 140.52 86.748984) (end 140.236992 87.031992) (width 0.254) (layer "B.Cu") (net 2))
 (segment (start 83.459141 87.979141) (end 83.459141 85.229994) (width 0.254) (layer "B.Cu") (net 2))
 (segment (start 140.236992 87.031992) (end 140.44 87.235) (width 0.254) (layer "B.Cu") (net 2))
 (segment (start 157.82 86.314336) (end 159.503722 84.630614) (width 0.254) (layer "B.Cu") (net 2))
 (segment (start 83.58 88.1) (end 83.58 88.093948) (width 0.2) (layer "B.Cu") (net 2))
 (segment (start 158.19163 88.997) (end 183.523 88.997) (width 0.254) (layer "B.Cu") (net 2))
 (segment (start 155.535664 86.314336) (end 157.82 86.314336) (width 0.508) (layer "B.Cu") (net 2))
 (segment (start 83.58 88.093948) (end 83.648008 88.02594) (width 0.2) (layer "B.Cu") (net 2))
 (segment (start 84.712068 89.09) (end 101.69 89.09) (width 0.254) (layer "B.Cu") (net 2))
 (segment (start 140.44 88.39) (end 137.310001 91.519999) (width 0.254) (layer "B.Cu") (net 2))
 (segment (start 108.29 87.9) (end 108.14295 87.9) (width 0.2) (layer "B.Cu") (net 2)))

